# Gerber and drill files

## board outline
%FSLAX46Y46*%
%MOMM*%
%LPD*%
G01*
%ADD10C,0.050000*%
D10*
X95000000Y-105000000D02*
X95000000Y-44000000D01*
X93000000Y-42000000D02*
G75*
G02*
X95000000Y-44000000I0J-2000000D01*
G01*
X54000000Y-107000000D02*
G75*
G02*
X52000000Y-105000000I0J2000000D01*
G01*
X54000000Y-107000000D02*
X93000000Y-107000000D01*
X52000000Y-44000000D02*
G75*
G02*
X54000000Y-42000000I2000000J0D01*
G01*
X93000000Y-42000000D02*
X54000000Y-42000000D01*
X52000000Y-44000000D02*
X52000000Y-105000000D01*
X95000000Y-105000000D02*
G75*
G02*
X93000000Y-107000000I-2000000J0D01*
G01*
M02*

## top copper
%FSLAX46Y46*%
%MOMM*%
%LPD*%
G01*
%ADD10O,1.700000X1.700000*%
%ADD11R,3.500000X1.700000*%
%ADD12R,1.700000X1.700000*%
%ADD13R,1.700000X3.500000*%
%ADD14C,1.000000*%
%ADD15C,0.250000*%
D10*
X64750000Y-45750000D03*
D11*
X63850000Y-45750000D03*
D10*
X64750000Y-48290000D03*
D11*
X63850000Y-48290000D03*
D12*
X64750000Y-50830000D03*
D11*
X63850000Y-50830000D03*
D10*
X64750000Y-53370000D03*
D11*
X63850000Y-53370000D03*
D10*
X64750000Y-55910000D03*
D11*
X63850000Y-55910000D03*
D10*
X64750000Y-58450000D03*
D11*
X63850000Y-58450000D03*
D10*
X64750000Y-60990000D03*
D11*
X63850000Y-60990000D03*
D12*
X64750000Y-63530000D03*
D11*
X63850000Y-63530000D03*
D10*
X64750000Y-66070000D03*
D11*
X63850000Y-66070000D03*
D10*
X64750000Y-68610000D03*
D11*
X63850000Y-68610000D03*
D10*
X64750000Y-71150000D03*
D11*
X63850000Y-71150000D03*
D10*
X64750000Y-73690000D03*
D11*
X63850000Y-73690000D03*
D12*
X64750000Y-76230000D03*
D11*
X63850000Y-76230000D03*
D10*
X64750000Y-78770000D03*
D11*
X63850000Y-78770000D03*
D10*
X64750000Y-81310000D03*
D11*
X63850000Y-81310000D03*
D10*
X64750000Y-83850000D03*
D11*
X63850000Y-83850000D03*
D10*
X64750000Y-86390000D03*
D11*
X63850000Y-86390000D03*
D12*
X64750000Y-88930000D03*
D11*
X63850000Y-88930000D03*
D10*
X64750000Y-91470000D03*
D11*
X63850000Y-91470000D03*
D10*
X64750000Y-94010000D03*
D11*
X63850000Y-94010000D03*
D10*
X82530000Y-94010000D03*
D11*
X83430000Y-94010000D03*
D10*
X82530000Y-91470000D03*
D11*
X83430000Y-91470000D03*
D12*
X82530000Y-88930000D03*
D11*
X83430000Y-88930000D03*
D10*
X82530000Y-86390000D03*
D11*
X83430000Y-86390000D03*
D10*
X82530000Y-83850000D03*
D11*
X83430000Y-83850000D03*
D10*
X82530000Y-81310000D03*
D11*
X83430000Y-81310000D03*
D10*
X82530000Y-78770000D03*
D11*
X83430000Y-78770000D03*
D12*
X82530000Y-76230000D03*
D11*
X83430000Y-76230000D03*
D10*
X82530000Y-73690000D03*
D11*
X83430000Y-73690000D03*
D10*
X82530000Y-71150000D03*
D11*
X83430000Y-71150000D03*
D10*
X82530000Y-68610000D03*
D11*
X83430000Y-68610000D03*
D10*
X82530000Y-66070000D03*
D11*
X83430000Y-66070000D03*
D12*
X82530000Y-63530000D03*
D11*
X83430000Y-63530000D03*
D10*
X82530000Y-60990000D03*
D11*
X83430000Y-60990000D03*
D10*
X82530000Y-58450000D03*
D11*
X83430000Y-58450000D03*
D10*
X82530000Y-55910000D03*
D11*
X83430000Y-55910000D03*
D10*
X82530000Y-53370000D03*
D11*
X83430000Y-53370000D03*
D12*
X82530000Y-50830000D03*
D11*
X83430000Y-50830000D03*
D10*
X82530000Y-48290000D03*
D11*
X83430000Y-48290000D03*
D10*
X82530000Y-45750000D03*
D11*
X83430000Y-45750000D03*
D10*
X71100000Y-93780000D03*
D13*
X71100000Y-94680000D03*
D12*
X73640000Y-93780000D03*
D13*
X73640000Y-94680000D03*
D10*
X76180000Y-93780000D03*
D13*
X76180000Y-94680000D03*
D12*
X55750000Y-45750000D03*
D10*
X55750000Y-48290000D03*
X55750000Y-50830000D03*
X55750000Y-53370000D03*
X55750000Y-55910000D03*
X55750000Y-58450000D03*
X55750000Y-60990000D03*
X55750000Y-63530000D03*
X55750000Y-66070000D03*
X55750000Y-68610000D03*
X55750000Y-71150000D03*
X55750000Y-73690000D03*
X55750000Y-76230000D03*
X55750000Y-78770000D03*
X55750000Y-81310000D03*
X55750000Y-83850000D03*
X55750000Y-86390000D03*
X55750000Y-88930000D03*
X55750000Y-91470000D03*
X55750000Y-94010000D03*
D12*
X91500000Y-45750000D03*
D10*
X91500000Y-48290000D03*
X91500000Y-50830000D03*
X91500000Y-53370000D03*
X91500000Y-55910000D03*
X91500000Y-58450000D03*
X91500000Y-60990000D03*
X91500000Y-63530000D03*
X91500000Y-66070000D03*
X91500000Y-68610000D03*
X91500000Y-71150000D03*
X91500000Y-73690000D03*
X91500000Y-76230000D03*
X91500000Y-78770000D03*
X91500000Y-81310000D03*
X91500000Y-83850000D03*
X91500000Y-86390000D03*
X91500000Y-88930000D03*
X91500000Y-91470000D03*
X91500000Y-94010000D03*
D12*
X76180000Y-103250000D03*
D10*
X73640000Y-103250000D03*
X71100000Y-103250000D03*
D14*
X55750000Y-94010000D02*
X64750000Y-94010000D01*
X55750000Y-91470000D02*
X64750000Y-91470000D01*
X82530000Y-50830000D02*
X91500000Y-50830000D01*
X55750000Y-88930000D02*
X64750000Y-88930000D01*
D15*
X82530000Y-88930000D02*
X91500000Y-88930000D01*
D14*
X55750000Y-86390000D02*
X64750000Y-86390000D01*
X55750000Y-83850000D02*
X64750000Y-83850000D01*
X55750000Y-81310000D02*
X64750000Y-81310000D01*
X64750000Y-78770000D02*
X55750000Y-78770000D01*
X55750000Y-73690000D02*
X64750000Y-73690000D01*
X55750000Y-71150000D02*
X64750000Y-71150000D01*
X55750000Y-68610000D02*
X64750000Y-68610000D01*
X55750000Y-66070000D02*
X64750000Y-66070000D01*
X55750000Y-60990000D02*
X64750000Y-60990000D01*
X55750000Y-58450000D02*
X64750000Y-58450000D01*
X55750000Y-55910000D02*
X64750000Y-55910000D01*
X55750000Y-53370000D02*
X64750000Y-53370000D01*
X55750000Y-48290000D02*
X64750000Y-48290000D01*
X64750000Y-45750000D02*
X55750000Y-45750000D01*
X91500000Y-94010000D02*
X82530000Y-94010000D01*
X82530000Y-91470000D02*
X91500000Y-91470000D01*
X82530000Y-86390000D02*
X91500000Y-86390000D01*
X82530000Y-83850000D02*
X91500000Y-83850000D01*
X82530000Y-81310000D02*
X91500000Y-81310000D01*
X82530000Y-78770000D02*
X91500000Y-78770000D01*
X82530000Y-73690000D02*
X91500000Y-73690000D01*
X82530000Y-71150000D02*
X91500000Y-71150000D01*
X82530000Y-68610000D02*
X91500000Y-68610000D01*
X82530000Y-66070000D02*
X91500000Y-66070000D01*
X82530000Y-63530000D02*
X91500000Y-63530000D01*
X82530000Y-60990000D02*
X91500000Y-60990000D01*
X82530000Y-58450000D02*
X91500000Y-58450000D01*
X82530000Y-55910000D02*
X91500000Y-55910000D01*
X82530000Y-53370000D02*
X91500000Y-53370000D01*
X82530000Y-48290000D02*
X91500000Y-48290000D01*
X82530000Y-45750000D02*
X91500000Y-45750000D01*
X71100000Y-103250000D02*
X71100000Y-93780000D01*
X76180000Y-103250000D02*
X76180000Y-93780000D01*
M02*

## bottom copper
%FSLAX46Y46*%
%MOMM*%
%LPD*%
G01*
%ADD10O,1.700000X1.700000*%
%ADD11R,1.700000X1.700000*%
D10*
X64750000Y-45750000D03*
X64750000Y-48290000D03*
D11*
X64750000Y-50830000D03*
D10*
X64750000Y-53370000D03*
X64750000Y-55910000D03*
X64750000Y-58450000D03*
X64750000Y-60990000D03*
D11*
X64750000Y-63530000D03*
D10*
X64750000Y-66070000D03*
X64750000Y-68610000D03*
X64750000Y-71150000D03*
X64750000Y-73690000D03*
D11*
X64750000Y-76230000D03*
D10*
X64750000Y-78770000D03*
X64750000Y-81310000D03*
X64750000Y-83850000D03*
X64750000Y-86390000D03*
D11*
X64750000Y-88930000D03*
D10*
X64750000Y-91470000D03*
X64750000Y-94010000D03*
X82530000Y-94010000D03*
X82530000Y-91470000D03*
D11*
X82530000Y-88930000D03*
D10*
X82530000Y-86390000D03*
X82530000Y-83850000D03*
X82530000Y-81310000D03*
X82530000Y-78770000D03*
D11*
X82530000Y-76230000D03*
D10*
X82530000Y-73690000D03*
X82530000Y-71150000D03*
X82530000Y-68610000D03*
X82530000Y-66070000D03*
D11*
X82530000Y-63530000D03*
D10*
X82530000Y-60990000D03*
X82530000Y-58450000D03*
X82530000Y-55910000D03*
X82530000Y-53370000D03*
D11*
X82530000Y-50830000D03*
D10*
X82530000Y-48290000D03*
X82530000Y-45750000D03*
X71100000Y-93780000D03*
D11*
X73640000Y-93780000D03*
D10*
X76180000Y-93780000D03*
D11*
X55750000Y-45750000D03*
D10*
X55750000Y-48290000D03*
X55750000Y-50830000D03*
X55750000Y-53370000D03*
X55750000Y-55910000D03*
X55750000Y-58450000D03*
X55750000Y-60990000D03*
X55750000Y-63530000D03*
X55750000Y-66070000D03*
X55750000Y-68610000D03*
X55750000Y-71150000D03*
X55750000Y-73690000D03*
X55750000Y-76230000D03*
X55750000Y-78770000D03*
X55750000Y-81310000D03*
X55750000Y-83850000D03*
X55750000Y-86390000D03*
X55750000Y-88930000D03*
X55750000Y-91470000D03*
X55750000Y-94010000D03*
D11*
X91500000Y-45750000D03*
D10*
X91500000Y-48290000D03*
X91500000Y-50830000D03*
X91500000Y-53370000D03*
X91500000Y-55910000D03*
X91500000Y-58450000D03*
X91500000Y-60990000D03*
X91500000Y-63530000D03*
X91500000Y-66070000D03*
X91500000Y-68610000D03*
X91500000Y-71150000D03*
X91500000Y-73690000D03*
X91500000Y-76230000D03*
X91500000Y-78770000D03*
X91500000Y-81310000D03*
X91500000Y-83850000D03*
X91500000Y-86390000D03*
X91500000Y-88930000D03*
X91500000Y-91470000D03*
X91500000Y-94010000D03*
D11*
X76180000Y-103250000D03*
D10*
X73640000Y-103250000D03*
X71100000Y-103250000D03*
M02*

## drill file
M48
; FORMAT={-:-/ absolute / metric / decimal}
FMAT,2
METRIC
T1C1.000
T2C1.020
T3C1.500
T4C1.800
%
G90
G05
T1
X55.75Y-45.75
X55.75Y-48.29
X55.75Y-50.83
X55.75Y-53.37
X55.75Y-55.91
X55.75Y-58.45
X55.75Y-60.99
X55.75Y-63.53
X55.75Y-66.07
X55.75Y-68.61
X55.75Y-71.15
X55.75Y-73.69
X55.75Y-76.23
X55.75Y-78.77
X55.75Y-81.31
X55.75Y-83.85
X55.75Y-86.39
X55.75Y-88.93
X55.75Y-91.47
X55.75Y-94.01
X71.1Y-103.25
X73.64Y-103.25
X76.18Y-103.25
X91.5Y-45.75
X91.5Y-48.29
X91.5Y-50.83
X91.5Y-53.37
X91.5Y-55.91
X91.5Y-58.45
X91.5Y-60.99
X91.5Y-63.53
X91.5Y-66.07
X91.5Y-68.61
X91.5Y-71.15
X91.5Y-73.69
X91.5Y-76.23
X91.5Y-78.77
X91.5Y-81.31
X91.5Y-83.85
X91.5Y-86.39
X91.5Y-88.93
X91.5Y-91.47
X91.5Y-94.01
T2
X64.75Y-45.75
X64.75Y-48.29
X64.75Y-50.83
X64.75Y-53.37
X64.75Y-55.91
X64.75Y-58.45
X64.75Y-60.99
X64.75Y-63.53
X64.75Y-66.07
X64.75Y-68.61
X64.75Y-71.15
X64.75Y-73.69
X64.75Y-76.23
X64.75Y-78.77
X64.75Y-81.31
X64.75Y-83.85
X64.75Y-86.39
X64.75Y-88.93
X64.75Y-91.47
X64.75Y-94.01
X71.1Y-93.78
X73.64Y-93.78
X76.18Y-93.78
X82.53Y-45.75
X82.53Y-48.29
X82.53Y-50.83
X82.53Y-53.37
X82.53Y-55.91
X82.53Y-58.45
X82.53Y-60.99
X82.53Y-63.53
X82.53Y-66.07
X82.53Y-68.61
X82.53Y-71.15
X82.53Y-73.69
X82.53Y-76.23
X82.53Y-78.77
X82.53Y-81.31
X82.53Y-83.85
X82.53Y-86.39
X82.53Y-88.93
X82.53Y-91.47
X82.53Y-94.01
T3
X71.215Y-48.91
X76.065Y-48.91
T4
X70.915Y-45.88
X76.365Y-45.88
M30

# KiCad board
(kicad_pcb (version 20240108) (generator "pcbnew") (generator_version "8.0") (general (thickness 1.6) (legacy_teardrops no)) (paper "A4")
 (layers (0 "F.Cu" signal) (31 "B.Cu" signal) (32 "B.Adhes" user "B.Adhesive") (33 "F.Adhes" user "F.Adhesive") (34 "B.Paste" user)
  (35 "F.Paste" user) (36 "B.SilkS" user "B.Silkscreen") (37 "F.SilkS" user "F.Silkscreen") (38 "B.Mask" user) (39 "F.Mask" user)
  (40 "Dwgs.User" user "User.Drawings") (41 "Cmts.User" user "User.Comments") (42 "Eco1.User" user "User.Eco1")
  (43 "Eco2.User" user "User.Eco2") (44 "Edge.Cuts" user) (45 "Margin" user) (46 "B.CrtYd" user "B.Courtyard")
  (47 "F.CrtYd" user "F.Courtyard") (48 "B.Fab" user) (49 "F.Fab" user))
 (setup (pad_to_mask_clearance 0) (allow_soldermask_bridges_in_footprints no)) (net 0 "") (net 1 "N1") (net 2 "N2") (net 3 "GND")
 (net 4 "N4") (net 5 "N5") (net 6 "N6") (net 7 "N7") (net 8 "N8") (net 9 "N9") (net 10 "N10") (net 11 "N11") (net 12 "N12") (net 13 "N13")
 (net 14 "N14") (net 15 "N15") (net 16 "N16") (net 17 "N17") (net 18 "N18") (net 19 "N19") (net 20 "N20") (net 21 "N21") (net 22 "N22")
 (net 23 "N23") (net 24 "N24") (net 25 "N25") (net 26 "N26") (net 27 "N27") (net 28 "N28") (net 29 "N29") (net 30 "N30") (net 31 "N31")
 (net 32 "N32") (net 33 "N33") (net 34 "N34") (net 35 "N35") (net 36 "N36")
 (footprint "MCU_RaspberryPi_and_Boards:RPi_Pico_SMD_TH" (layer "F.Cu") (at 73.64 69.88)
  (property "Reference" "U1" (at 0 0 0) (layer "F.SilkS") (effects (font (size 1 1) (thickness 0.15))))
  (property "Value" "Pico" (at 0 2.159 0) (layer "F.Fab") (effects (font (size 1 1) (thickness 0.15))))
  (pad "" np_thru_hole oval (at -2.725 -24) (size 1.8 1.8) (drill 1.8) (layers "*.Cu" "*.Mask"))
  (pad "" np_thru_hole oval (at -2.425 -20.97) (size 1.5 1.5) (drill 1.5) (layers "*.Cu" "*.Mask"))
  (pad "" np_thru_hole oval (at 2.425 -20.97) (size 1.5 1.5) (drill 1.5) (layers "*.Cu" "*.Mask"))
  (pad "" np_thru_hole oval (at 2.725 -24) (size 1.8 1.8) (drill 1.8) (layers "*.Cu" "*.Mask"))
  (pad "1" thru_hole oval (at -8.89 -24.13) (size 1.7 1.7) (drill 1.02) (layers "*.Cu" "*.Mask") (remove_unused_layers no) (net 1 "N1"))
  (pad "1" smd rect (at -8.89 -24.13) (size 3.5 1.7) (drill (offset -0.9 0)) (layers "F.Cu" "F.Mask") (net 1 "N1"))
  (pad "2" thru_hole oval (at -8.89 -21.59) (size 1.7 1.7) (drill 1.02) (layers "*.Cu" "*.Mask") (remove_unused_layers no) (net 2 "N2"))
  (pad "2" smd rect (at -8.89 -21.59) (size 3.5 1.7) (drill (offset -0.9 0)) (layers "F.Cu" "F.Mask") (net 2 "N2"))
  (pad "3" thru_hole rect (at -8.89 -19.05) (size 1.7 1.7) (drill 1.02) (layers "*.Cu" "*.Mask") (remove_unused_layers no) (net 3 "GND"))
  (pad "3" smd rect (at -8.89 -19.05) (size 3.5 1.7) (drill (offset -0.9 0)) (layers "F.Cu" "F.Mask") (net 3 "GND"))
  (pad "4" thru_hole oval (at -8.89 -16.51) (size 1.7 1.7) (drill 1.02) (layers "*.Cu" "*.Mask") (remove_unused_layers no) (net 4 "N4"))
  (pad "4" smd rect (at -8.89 -16.51) (size 3.5 1.7) (drill (offset -0.9 0)) (layers "F.Cu" "F.Mask") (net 4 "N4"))
  (pad "5" thru_hole oval (at -8.89 -13.97) (size 1.7 1.7) (drill 1.02) (layers "*.Cu" "*.Mask") (remove_unused_layers no) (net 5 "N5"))
  (pad "5" smd rect (at -8.89 -13.97) (size 3.5 1.7) (drill (offset -0.9 0)) (layers "F.Cu" "F.Mask") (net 5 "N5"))
  (pad "6" thru_hole oval (at -8.89 -11.43) (size 1.7 1.7) (drill 1.02) (layers "*.Cu" "*.Mask") (remove_unused_layers no) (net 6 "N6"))
  (pad "6" smd rect (at -8.89 -11.43) (size 3.5 1.7) (drill (offset -0.9 0)) (layers "F.Cu" "F.Mask") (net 6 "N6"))
  (pad "7" thru_hole oval (at -8.89 -8.89) (size 1.7 1.7) (drill 1.02) (layers "*.Cu" "*.Mask") (remove_unused_layers no) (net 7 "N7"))
  (pad "7" smd rect (at -8.89 -8.89) (size 3.5 1.7) (drill (offset -0.9 0)) (layers "F.Cu" "F.Mask") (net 7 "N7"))
  (pad "8" thru_hole rect (at -8.89 -6.35) (size 1.7 1.7) (drill 1.02) (layers "*.Cu" "*.Mask") (remove_unused_layers no) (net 3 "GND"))
  (pad "8" smd rect (at -8.89 -6.35) (size 3.5 1.7) (drill (offset -0.9 0)) (layers "F.Cu" "F.Mask") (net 3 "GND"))
  (pad "9" thru_hole oval (at -8.89 -3.81) (size 1.7 1.7) (drill 1.02) (layers "*.Cu" "*.Mask") (remove_unused_layers no) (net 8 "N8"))
  (pad "9" smd rect (at -8.89 -3.81) (size 3.5 1.7) (drill (offset -0.9 0)) (layers "F.Cu" "F.Mask") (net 8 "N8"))
  (pad "10" thru_hole oval (at -8.89 -1.27) (size 1.7 1.7) (drill 1.02) (layers "*.Cu" "*.Mask") (remove_unused_layers no) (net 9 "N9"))
  (pad "10" smd rect (at -8.89 -1.27) (size 3.5 1.7) (drill (offset -0.9 0)) (layers "F.Cu" "F.Mask") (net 9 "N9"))
  (pad "11" thru_hole oval (at -8.89 1.27) (size 1.7 1.7) (drill 1.02) (layers "*.Cu" "*.Mask") (remove_unused_layers no) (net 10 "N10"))
  (pad "11" smd rect (at -8.89 1.27) (size 3.5 1.7) (drill (offset -0.9 0)) (layers "F.Cu" "F.Mask") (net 10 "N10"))
  (pad "12" thru_hole oval (at -8.89 3.81) (size 1.7 1.7) (drill 1.02) (layers "*.Cu" "*.Mask") (remove_unused_layers no) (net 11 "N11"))
  (pad "12" smd rect (at -8.89 3.81) (size 3.5 1.7) (drill (offset -0.9 0)) (layers "F.Cu" "F.Mask") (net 11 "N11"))
  (pad "13" thru_hole rect (at -8.89 6.35) (size 1.7 1.7) (drill 1.02) (layers "*.Cu" "*.Mask") (remove_unused_layers no) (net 3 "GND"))
  (pad "13" smd rect (at -8.89 6.35) (size 3.5 1.7) (drill (offset -0.9 0)) (layers "F.Cu" "F.Mask") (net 3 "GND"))
  (pad "14" thru_hole oval (at -8.89 8.89) (size 1.7 1.7) (drill 1.02) (layers "*.Cu" "*.Mask") (remove_unused_layers no) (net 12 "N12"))
  (pad "14" smd rect (at -8.89 8.89) (size 3.5 1.7) (drill (offset -0.9 0)) (layers "F.Cu" "F.Mask") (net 12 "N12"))
  (pad "15" thru_hole oval (at -8.89 11.43) (size 1.7 1.7) (drill 1.02) (layers "*.Cu" "*.Mask") (remove_unused_layers no) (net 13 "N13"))
  (pad "15" smd rect (at -8.89 11.43) (size 3.5 1.7) (drill (offset -0.9 0)) (layers "F.Cu" "F.Mask") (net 13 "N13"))
  (pad "16" thru_hole oval (at -8.89 13.97) (size 1.7 1.7) (drill 1.02) (layers "*.Cu" "*.Mask") (remove_unused_layers no) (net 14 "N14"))
  (pad "16" smd rect (at -8.89 13.97) (size 3.5 1.7) (drill (offset -0.9 0)) (layers "F.Cu" "F.Mask") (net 14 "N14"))
  (pad "17" thru_hole oval (at -8.89 16.51) (size 1.7 1.7) (drill 1.02) (layers "*.Cu" "*.Mask") (remove_unused_layers no) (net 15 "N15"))
  (pad "17" smd rect (at -8.89 16.51) (size 3.5 1.7) (drill (offset -0.9 0)) (layers "F.Cu" "F.Mask") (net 15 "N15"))
  (pad "18" thru_hole rect (at -8.89 19.05) (size 1.7 1.7) (drill 1.02) (layers "*.Cu" "*.Mask") (remove_unused_layers no) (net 3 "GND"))
  (pad "18" smd rect (at -8.89 19.05) (size 3.5 1.7) (drill (offset -0.9 0)) (layers "F.Cu" "F.Mask") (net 3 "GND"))
  (pad "19" thru_hole oval (at -8.89 21.59) (size 1.7 1.7) (drill 1.02) (layers "*.Cu" "*.Mask") (remove_unused_layers no) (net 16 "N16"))
  (pad "19" smd rect (at -8.89 21.59) (size 3.5 1.7) (drill (offset -0.9 0)) (layers "F.Cu" "F.Mask") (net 16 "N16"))
  (pad "20" thru_hole oval (at -8.89 24.13) (size 1.7 1.7) (drill 1.02) (layers "*.Cu" "*.Mask") (remove_unused_layers no) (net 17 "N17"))
  (pad "20" smd rect (at -8.89 24.13) (size 3.5 1.7) (drill (offset -0.9 0)) (layers "F.Cu" "F.Mask") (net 17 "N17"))
  (pad "21" thru_hole oval (at 8.89 24.13) (size 1.7 1.7) (drill 1.02) (layers "*.Cu" "*.Mask") (remove_unused_layers no) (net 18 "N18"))
  (pad "21" smd rect (at 8.89 24.13) (size 3.5 1.7) (drill (offset 0.9 0)) (layers "F.Cu" "F.Mask") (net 18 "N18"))
  (pad "22" thru_hole oval (at 8.89 21.59) (size 1.7 1.7) (drill 1.02) (layers "*.Cu" "*.Mask") (remove_unused_layers no) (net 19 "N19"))
  (pad "22" smd rect (at 8.89 21.59) (size 3.5 1.7) (drill (offset 0.9 0)) (layers "F.Cu" "F.Mask") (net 19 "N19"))
  (pad "23" thru_hole rect (at 8.89 19.05) (size 1.7 1.7) (drill 1.02) (layers "*.Cu" "*.Mask") (remove_unused_layers no) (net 3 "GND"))
  (pad "23" smd rect (at 8.89 19.05) (size 3.5 1.7) (drill (offset 0.9 0)) (layers "F.Cu" "F.Mask") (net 3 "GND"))
  (pad "24" thru_hole oval (at 8.89 16.51) (size 1.7 1.7) (drill 1.02) (layers "*.Cu" "*.Mask") (remove_unused_layers no) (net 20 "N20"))
  (pad "24" smd rect (at 8.89 16.51) (size 3.5 1.7) (drill (offset 0.9 0)) (layers "F.Cu" "F.Mask") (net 20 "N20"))
  (pad "25" thru_hole oval (at 8.89 13.97) (size 1.7 1.7) (drill 1.02) (layers "*.Cu" "*.Mask") (remove_unused_layers no) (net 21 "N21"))
  (pad "25" smd rect (at 8.89 13.97) (size 3.5 1.7) (drill (offset 0.9 0)) (layers "F.Cu" "F.Mask") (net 21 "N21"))
  (pad "26" thru_hole oval (at 8.89 11.43) (size 1.7 1.7) (drill 1.02) (layers "*.Cu" "*.Mask") (remove_unused_layers no) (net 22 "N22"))
  (pad "26" smd rect (at 8.89 11.43) (size 3.5 1.7) (drill (offset 0.9 0)) (layers "F.Cu" "F.Mask") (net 22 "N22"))
  (pad "27" thru_hole oval (at 8.89 8.89) (size 1.7 1.7) (drill 1.02) (layers "*.Cu" "*.Mask") (remove_unused_layers no) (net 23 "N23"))
  (pad "27" smd rect (at 8.89 8.89) (size 3.5 1.7) (drill (offset 0.9 0)) (layers "F.Cu" "F.Mask") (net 23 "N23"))
  (pad "28" thru_hole rect (at 8.89 6.35) (size 1.7 1.7) (drill 1.02) (layers "*.Cu" "*.Mask") (remove_unused_layers no) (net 3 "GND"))
  (pad "28" smd rect (at 8.89 6.35) (size 3.5 1.7) (drill (offset 0.9 0)) (layers "F.Cu" "F.Mask") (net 3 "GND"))
  (pad "29" thru_hole oval (at 8.89 3.81) (size 1.7 1.7) (drill 1.02) (layers "*.Cu" "*.Mask") (remove_unused_layers no) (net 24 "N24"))
  (pad "29" smd rect (at 8.89 3.81) (size 3.5 1.7) (drill (offset 0.9 0)) (layers "F.Cu" "F.Mask") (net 24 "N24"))
  (pad "30" thru_hole oval (at 8.89 1.27) (size 1.7 1.7) (drill 1.02) (layers "*.Cu" "*.Mask") (remove_unused_layers no) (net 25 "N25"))
  (pad "30" smd rect (at 8.89 1.27) (size 3.5 1.7) (drill (offset 0.9 0)) (layers "F.Cu" "F.Mask") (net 25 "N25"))
  (pad "31" thru_hole oval (at 8.89 -1.27) (size 1.7 1.7) (drill 1.02) (layers "*.Cu" "*.Mask") (remove_unused_layers no) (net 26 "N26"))
  (pad "31" smd rect (at 8.89 -1.27) (size 3.5 1.7) (drill (offset 0.9 0)) (layers "F.Cu" "F.Mask") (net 26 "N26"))
  (pad "32" thru_hole oval (at 8.89 -3.81) (size 1.7 1.7) (drill 1.02) (layers "*.Cu" "*.Mask") (remove_unused_layers no) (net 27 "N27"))
  (pad "32" smd rect (at 8.89 -3.81) (size 3.5 1.7) (drill (offset 0.9 0)) (layers "F.Cu" "F.Mask") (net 27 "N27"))
  (pad "33" thru_hole rect (at 8.89 -6.35) (size 1.7 1.7) (drill 1.02) (layers "*.Cu" "*.Mask") (remove_unused_layers no) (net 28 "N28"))
  (pad "33" smd rect (at 8.89 -6.35) (size 3.5 1.7) (drill (offset 0.9 0)) (layers "F.Cu" "F.Mask") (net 28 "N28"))
  (pad "34" thru_hole oval (at 8.89 -8.89) (size 1.7 1.7) (drill 1.02) (layers "*.Cu" "*.Mask") (remove_unused_layers no) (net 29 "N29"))
  (pad "34" smd rect (at 8.89 -8.89) (size 3.5 1.7) (drill (offset 0.9 0)) (layers "F.Cu" "F.Mask") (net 29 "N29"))
  (pad "35" thru_hole oval (at 8.89 -11.43) (size 1.7 1.7) (drill 1.02) (layers "*.Cu" "*.Mask") (remove_unused_layers no) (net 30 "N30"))
  (pad "35" smd rect (at 8.89 -11.43) (size 3.5 1.7) (drill (offset 0.9 0)) (layers "F.Cu" "F.Mask") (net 30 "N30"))
  (pad "36" thru_hole oval (at 8.89 -13.97) (size 1.7 1.7) (drill 1.02) (layers "*.Cu" "*.Mask") (remove_unused_layers no) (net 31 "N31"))
  (pad "36" smd rect (at 8.89 -13.97) (size 3.5 1.7) (drill (offset 0.9 0)) (layers "F.Cu" "F.Mask") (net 31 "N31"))
  (pad "37" thru_hole oval (at 8.89 -16.51) (size 1.7 1.7) (drill 1.02) (layers "*.Cu" "*.Mask") (remove_unused_layers no) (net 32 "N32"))
  (pad "37" smd rect (at 8.89 -16.51) (size 3.5 1.7) (drill (offset 0.9 0)) (layers "F.Cu" "F.Mask") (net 32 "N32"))
  (pad "38" thru_hole rect (at 8.89 -19.05) (size 1.7 1.7) (drill 1.02) (layers "*.Cu" "*.Mask") (remove_unused_layers no) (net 3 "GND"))
  (pad "38" smd rect (at 8.89 -19.05) (size 3.5 1.7) (drill (offset 0.9 0)) (layers "F.Cu" "F.Mask") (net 3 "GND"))
  (pad "39" thru_hole oval (at 8.89 -21.59) (size 1.7 1.7) (drill 1.02) (layers "*.Cu" "*.Mask") (remove_unused_layers no) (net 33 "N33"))
  (pad "39" smd rect (at 8.89 -21.59) (size 3.5 1.7) (drill (offset 0.9 0)) (layers "F.Cu" "F.Mask") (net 33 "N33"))
  (pad "40" thru_hole oval (at 8.89 -24.13) (size 1.7 1.7) (drill 1.02) (layers "*.Cu" "*.Mask") (remove_unused_layers no) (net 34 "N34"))
  (pad "40" smd rect (at 8.89 -24.13) (size 3.5 1.7) (drill (offset 0.9 0)) (layers "F.Cu" "F.Mask") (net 34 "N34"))
  (pad "41" thru_hole oval (at -2.54 23.9) (size 1.7 1.7) (drill 1.02) (layers "*.Cu" "*.Mask") (remove_unused_layers no) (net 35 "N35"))
  (pad "41" smd rect (at -2.54 23.9 90) (size 3.5 1.7) (drill (offset -0.9 0)) (layers "F.Cu" "F.Mask") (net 35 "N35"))
  (pad "42" thru_hole rect (at 0 23.9) (size 1.7 1.7) (drill 1.02) (layers "*.Cu" "*.Mask") (remove_unused_layers no) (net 3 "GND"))
  (pad "42" smd rect (at 0 23.9 90) (size 3.5 1.7) (drill (offset -0.9 0)) (layers "F.Cu" "F.Mask") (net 3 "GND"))
  (pad "43" thru_hole oval (at 2.54 23.9) (size 1.7 1.7) (drill 1.02) (layers "*.Cu" "*.Mask") (remove_unused_layers no) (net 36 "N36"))
  (pad "43" smd rect (at 2.54 23.9 90) (size 3.5 1.7) (drill (offset -0.9 0)) (layers "F.Cu" "F.Mask") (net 36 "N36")))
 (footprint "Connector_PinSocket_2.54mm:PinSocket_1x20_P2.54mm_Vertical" (layer "F.Cu") (at 55.75 45.75)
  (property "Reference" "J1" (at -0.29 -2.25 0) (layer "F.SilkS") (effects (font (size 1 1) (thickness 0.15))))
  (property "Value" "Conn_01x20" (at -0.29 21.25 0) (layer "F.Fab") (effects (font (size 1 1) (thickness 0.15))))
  (pad "1" thru_hole rect (at 0 0) (size 1.7 1.7) (drill 1) (layers "*.Cu" "*.Mask") (remove_unused_layers no) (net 1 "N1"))
  (pad "2" thru_hole oval (at 0 2.54) (size 1.7 1.7) (drill 1) (layers "*.Cu" "*.Mask") (remove_unused_layers no) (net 2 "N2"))
  (pad "3" thru_hole oval (at 0 5.08) (size 1.7 1.7) (drill 1) (layers "*.Cu" "*.Mask") (remove_unused_layers no) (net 3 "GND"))
  (pad "4" thru_hole oval (at 0 7.62) (size 1.7 1.7) (drill 1) (layers "*.Cu" "*.Mask") (remove_unused_layers no) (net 4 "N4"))
  (pad "5" thru_hole oval (at 0 10.16) (size 1.7 1.7) (drill 1) (layers "*.Cu" "*.Mask") (remove_unused_layers no) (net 5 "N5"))
  (pad "6" thru_hole oval (at 0 12.7) (size 1.7 1.7) (drill 1) (layers "*.Cu" "*.Mask") (remove_unused_layers no) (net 6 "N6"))
  (pad "7" thru_hole oval (at 0 15.24) (size 1.7 1.7) (drill 1) (layers "*.Cu" "*.Mask") (remove_unused_layers no) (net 7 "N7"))
  (pad "8" thru_hole oval (at 0 17.78) (size 1.7 1.7) (drill 1) (layers "*.Cu" "*.Mask") (remove_unused_layers no) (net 3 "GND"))
  (pad "9" thru_hole oval (at 0 20.32) (size 1.7 1.7) (drill 1) (layers "*.Cu" "*.Mask") (remove_unused_layers no) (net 8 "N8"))
  (pad "10" thru_hole oval (at 0 22.86) (size 1.7 1.7) (drill 1) (layers "*.Cu" "*.Mask") (remove_unused_layers no) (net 9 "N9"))
  (pad "11" thru_hole oval (at 0 25.4) (size 1.7 1.7) (drill 1) (layers "*.Cu" "*.Mask") (remove_unused_layers no) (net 10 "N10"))
  (pad "12" thru_hole oval (at 0 27.94) (size 1.7 1.7) (drill 1) (layers "*.Cu" "*.Mask") (remove_unused_layers no) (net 11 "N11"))
  (pad "13" thru_hole oval (at 0 30.48) (size 1.7 1.7) (drill 1) (layers "*.Cu" "*.Mask") (remove_unused_layers no) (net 3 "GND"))
  (pad "14" thru_hole oval (at 0 33.02) (size 1.7 1.7) (drill 1) (layers "*.Cu" "*.Mask") (remove_unused_layers no) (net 12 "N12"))
  (pad "15" thru_hole oval (at 0 35.56) (size 1.7 1.7) (drill 1) (layers "*.Cu" "*.Mask") (remove_unused_layers no) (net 13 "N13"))
  (pad "16" thru_hole oval (at 0 38.1) (size 1.7 1.7) (drill 1) (layers "*.Cu" "*.Mask") (remove_unused_layers no) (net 14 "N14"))
  (pad "17" thru_hole oval (at 0 40.64) (size 1.7 1.7) (drill 1) (layers "*.Cu" "*.Mask") (remove_unused_layers no) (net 15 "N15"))
  (pad "18" thru_hole oval (at 0 43.18) (size 1.7 1.7) (drill 1) (layers "*.Cu" "*.Mask") (remove_unused_layers no) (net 3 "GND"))
  (pad "19" thru_hole oval (at 0 45.72) (size 1.7 1.7) (drill 1) (layers "*.Cu" "*.Mask") (remove_unused_layers no) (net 16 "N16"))
  (pad "20" thru_hole oval (at 0 48.26) (size 1.7 1.7) (drill 1) (layers "*.Cu" "*.Mask") (remove_unused_layers no) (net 17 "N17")))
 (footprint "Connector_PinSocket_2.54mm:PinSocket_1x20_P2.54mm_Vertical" (layer "F.Cu") (at 91.5 45.75)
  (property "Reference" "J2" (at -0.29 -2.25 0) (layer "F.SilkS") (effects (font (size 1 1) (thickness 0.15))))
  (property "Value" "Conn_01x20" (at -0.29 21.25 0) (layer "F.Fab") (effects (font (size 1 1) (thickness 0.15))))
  (pad "1" thru_hole rect (at 0 0) (size 1.7 1.7) (drill 1) (layers "*.Cu" "*.Mask") (remove_unused_layers no) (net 34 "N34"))
  (pad "2" thru_hole oval (at 0 2.54) (size 1.7 1.7) (drill 1) (layers "*.Cu" "*.Mask") (remove_unused_layers no) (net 33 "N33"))
  (pad "3" thru_hole oval (at 0 5.08) (size 1.7 1.7) (drill 1) (layers "*.Cu" "*.Mask") (remove_unused_layers no) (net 3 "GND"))
  (pad "4" thru_hole oval (at 0 7.62) (size 1.7 1.7) (drill 1) (layers "*.Cu" "*.Mask") (remove_unused_layers no) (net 32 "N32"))
  (pad "5" thru_hole oval (at 0 10.16) (size 1.7 1.7) (drill 1) (layers "*.Cu" "*.Mask") (remove_unused_layers no) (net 31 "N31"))
  (pad "6" thru_hole oval (at 0 12.7) (size 1.7 1.7) (drill 1) (layers "*.Cu" "*.Mask") (remove_unused_layers no) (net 30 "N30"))
  (pad "7" thru_hole oval (at 0 15.24) (size 1.7 1.7) (drill 1) (layers "*.Cu" "*.Mask") (remove_unused_layers no) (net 29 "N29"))
  (pad "8" thru_hole oval (at 0 17.78) (size 1.7 1.7) (drill 1) (layers "*.Cu" "*.Mask") (remove_unused_layers no) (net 28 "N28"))
  (pad "9" thru_hole oval (at 0 20.32) (size 1.7 1.7) (drill 1) (layers "*.Cu" "*.Mask") (remove_unused_layers no) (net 27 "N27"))
  (pad "10" thru_hole oval (at 0 22.86) (size 1.7 1.7) (drill 1) (layers "*.Cu" "*.Mask") (remove_unused_layers no) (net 26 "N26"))
  (pad "11" thru_hole oval (at 0 25.4) (size 1.7 1.7) (drill 1) (layers "*.Cu" "*.Mask") (remove_unused_layers no) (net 25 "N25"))
  (pad "12" thru_hole oval (at 0 27.94) (size 1.7 1.7) (drill 1) (layers "*.Cu" "*.Mask") (remove_unused_layers no) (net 24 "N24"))
  (pad "13" thru_hole oval (at 0 30.48) (size 1.7 1.7) (drill 1) (layers "*.Cu" "*.Mask") (remove_unused_layers no) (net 3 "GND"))
  (pad "14" thru_hole oval (at 0 33.02) (size 1.7 1.7) (drill 1) (layers "*.Cu" "*.Mask") (remove_unused_layers no) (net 23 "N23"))
  (pad "15" thru_hole oval (at 0 35.56) (size 1.7 1.7) (drill 1) (layers "*.Cu" "*.Mask") (remove_unused_layers no) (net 22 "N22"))
  (pad "16" thru_hole oval (at 0 38.1) (size 1.7 1.7) (drill 1) (layers "*.Cu" "*.Mask") (remove_unused_layers no) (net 21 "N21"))
  (pad "17" thru_hole oval (at 0 40.64) (size 1.7 1.7) (drill 1) (layers "*.Cu" "*.Mask") (remove_unused_layers no) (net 20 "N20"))
  (pad "18" thru_hole oval (at 0 43.18) (size 1.7 1.7) (drill 1) (layers "*.Cu" "*.Mask") (remove_unused_layers no) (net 3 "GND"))
  (pad "19" thru_hole oval (at 0 45.72) (size 1.7 1.7) (drill 1) (layers "*.Cu" "*.Mask") (remove_unused_layers no) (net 19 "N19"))
  (pad "20" thru_hole oval (at 0 48.26) (size 1.7 1.7) (drill 1) (layers "*.Cu" "*.Mask") (remove_unused_layers no) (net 18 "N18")))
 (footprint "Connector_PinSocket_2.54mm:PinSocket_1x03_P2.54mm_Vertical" (layer "F.Cu") (at 76.18 103.25 -90)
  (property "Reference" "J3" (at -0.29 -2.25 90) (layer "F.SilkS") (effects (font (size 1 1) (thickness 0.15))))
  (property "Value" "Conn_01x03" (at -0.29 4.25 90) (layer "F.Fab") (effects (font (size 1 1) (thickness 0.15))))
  (pad "1" thru_hole rect (at 0 0 270) (size 1.7 1.7) (drill 1) (layers "*.Cu" "*.Mask") (remove_unused_layers no) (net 36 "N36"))
  (pad "2" thru_hole oval (at 0 2.54 270) (size 1.7 1.7) (drill 1) (layers "*.Cu" "*.Mask") (remove_unused_layers no) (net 3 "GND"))
  (pad "3" thru_hole oval (at 0 5.08 270) (size 1.7 1.7) (drill 1) (layers "*.Cu" "*.Mask") (remove_unused_layers no) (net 35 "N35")))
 (gr_line (start 95 105) (end 95 44) (stroke (width 0.05) (type solid)) (layer "Edge.Cuts"))
 (gr_arc (start 93 42) (mid 94.414214 42.585786) (end 95 44) (stroke (width 0.05) (type solid)) (layer "Edge.Cuts"))
 (gr_arc (start 54 107) (mid 52.585786 106.414214) (end 52 105) (stroke (width 0.05) (type solid)) (layer "Edge.Cuts"))
 (gr_line (start 54 107) (end 93 107) (stroke (width 0.05) (type solid)) (layer "Edge.Cuts"))
 (gr_arc (start 52 44) (mid 52.585786 42.585786) (end 54 42) (stroke (width 0.05) (type solid)) (layer "Edge.Cuts"))
 (gr_line (start 93 42) (end 54 42) (stroke (width 0.05) (type solid)) (layer "Edge.Cuts"))
 (gr_line (start 52 44) (end 52 105) (stroke (width 0.05) (type solid)) (layer "Edge.Cuts"))
 (gr_arc (start 95 105) (mid 94.414214 106.414214) (end 93 107) (stroke (width 0.05) (type solid)) (layer "Edge.Cuts"))
 (segment (start 55.75 94.01) (end 64.75 94.01) (width 1) (layer "F.Cu") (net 17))
 (segment (start 55.75 91.47) (end 64.75 91.47) (width 1) (layer "F.Cu") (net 16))
 (segment (start 82.53 50.83) (end 91.5 50.83) (width 1) (layer "F.Cu") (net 3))
 (segment (start 55.75 88.93) (end 64.75 88.93) (width 1) (layer "F.Cu") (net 3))
 (segment (start 82.53 88.93) (end 91.5 88.93) (width 0.25) (layer "F.Cu") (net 3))
 (segment (start 55.75 86.39) (end 64.75 86.39) (width 1) (layer "F.Cu") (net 15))
 (segment (start 55.75 83.85) (end 64.75 83.85) (width 1) (layer "F.Cu") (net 14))
 (segment (start 55.75 81.31) (end 64.75 81.31) (width 1) (layer "F.Cu") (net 13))
 (segment (start 64.75 78.77) (end 55.75 78.77) (width 1) (layer "F.Cu") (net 12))
 (segment (start 55.75 73.69) (end 64.75 73.69) (width 1) (layer "F.Cu") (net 11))
 (segment (start 55.75 71.15) (end 64.75 71.15) (width 1) (layer "F.Cu") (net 10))
 (segment (start 55.75 68.61) (end 64.75 68.61) (width 1) (layer "F.Cu") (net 9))
 (segment (start 55.75 66.07) (end 64.75 66.07) (width 1) (layer "F.Cu") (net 8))
 (segment (start 55.75 60.99) (end 64.75 60.99) (width 1) (layer "F.Cu") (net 7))
 (segment (start 55.75 58.45) (end 64.75 58.45) (width 1) (layer "F.Cu") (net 6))
 (segment (start 55.75 55.91) (end 64.75 55.91) (width 1) (layer "F.Cu") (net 5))
 (segment (start 55.75 53.37) (end 64.75 53.37) (width 1) (layer "F.Cu") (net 4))
 (segment (start 55.75 48.29) (end 64.75 48.29) (width 1) (layer "F.Cu") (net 2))
 (segment (start 64.75 45.75) (end 55.75 45.75) (width 1) (layer "F.Cu") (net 1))
 (segment (start 91.5 94.01) (end 82.53 94.01) (width 1) (layer "F.Cu") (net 18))
 (segment (start 82.53 91.47) (end 91.5 91.47) (width 1) (layer "F.Cu") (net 19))
 (segment (start 82.53 86.39) (end 91.5 86.39) (width 1) (layer "F.Cu") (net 20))
 (segment (start 82.53 83.85) (end 91.5 83.85) (width 1) (layer "F.Cu") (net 21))
 (segment (start 82.53 81.31) (end 91.5 81.31) (width 1) (layer "F.Cu") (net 22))
 (segment (start 82.53 78.77) (end 91.5 78.77) (width 1) (layer "F.Cu") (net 23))
 (segment (start 82.53 73.69) (end 91.5 73.69) (width 1) (layer "F.Cu") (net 24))
 (segment (start 82.53 71.15) (end 91.5 71.15) (width 1) (layer "F.Cu") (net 25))
 (segment (start 82.53 68.61) (end 91.5 68.61) (width 1) (layer "F.Cu") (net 26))
 (segment (start 82.53 66.07) (end 91.5 66.07) (width 1) (layer "F.Cu") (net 27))
 (segment (start 82.53 63.53) (end 91.5 63.53) (width 1) (layer "F.Cu") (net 28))
 (segment (start 82.53 60.99) (end 91.5 60.99) (width 1) (layer "F.Cu") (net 29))
 (segment (start 82.53 58.45) (end 91.5 58.45) (width 1) (layer "F.Cu") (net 30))
 (segment (start 82.53 55.91) (end 91.5 55.91) (width 1) (layer "F.Cu") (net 31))
 (segment (start 82.53 53.37) (end 91.5 53.37) (width 1) (layer "F.Cu") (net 32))
 (segment (start 82.53 48.29) (end 91.5 48.29) (width 1) (layer "F.Cu") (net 33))
 (segment (start 82.53 45.75) (end 91.5 45.75) (width 1) (layer "F.Cu") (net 34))
 (segment (start 71.1 103.25) (end 71.1 93.78) (width 1) (layer "F.Cu") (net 35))
 (segment (start 76.18 103.25) (end 76.18 93.78) (width 1) (layer "F.Cu") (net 36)))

